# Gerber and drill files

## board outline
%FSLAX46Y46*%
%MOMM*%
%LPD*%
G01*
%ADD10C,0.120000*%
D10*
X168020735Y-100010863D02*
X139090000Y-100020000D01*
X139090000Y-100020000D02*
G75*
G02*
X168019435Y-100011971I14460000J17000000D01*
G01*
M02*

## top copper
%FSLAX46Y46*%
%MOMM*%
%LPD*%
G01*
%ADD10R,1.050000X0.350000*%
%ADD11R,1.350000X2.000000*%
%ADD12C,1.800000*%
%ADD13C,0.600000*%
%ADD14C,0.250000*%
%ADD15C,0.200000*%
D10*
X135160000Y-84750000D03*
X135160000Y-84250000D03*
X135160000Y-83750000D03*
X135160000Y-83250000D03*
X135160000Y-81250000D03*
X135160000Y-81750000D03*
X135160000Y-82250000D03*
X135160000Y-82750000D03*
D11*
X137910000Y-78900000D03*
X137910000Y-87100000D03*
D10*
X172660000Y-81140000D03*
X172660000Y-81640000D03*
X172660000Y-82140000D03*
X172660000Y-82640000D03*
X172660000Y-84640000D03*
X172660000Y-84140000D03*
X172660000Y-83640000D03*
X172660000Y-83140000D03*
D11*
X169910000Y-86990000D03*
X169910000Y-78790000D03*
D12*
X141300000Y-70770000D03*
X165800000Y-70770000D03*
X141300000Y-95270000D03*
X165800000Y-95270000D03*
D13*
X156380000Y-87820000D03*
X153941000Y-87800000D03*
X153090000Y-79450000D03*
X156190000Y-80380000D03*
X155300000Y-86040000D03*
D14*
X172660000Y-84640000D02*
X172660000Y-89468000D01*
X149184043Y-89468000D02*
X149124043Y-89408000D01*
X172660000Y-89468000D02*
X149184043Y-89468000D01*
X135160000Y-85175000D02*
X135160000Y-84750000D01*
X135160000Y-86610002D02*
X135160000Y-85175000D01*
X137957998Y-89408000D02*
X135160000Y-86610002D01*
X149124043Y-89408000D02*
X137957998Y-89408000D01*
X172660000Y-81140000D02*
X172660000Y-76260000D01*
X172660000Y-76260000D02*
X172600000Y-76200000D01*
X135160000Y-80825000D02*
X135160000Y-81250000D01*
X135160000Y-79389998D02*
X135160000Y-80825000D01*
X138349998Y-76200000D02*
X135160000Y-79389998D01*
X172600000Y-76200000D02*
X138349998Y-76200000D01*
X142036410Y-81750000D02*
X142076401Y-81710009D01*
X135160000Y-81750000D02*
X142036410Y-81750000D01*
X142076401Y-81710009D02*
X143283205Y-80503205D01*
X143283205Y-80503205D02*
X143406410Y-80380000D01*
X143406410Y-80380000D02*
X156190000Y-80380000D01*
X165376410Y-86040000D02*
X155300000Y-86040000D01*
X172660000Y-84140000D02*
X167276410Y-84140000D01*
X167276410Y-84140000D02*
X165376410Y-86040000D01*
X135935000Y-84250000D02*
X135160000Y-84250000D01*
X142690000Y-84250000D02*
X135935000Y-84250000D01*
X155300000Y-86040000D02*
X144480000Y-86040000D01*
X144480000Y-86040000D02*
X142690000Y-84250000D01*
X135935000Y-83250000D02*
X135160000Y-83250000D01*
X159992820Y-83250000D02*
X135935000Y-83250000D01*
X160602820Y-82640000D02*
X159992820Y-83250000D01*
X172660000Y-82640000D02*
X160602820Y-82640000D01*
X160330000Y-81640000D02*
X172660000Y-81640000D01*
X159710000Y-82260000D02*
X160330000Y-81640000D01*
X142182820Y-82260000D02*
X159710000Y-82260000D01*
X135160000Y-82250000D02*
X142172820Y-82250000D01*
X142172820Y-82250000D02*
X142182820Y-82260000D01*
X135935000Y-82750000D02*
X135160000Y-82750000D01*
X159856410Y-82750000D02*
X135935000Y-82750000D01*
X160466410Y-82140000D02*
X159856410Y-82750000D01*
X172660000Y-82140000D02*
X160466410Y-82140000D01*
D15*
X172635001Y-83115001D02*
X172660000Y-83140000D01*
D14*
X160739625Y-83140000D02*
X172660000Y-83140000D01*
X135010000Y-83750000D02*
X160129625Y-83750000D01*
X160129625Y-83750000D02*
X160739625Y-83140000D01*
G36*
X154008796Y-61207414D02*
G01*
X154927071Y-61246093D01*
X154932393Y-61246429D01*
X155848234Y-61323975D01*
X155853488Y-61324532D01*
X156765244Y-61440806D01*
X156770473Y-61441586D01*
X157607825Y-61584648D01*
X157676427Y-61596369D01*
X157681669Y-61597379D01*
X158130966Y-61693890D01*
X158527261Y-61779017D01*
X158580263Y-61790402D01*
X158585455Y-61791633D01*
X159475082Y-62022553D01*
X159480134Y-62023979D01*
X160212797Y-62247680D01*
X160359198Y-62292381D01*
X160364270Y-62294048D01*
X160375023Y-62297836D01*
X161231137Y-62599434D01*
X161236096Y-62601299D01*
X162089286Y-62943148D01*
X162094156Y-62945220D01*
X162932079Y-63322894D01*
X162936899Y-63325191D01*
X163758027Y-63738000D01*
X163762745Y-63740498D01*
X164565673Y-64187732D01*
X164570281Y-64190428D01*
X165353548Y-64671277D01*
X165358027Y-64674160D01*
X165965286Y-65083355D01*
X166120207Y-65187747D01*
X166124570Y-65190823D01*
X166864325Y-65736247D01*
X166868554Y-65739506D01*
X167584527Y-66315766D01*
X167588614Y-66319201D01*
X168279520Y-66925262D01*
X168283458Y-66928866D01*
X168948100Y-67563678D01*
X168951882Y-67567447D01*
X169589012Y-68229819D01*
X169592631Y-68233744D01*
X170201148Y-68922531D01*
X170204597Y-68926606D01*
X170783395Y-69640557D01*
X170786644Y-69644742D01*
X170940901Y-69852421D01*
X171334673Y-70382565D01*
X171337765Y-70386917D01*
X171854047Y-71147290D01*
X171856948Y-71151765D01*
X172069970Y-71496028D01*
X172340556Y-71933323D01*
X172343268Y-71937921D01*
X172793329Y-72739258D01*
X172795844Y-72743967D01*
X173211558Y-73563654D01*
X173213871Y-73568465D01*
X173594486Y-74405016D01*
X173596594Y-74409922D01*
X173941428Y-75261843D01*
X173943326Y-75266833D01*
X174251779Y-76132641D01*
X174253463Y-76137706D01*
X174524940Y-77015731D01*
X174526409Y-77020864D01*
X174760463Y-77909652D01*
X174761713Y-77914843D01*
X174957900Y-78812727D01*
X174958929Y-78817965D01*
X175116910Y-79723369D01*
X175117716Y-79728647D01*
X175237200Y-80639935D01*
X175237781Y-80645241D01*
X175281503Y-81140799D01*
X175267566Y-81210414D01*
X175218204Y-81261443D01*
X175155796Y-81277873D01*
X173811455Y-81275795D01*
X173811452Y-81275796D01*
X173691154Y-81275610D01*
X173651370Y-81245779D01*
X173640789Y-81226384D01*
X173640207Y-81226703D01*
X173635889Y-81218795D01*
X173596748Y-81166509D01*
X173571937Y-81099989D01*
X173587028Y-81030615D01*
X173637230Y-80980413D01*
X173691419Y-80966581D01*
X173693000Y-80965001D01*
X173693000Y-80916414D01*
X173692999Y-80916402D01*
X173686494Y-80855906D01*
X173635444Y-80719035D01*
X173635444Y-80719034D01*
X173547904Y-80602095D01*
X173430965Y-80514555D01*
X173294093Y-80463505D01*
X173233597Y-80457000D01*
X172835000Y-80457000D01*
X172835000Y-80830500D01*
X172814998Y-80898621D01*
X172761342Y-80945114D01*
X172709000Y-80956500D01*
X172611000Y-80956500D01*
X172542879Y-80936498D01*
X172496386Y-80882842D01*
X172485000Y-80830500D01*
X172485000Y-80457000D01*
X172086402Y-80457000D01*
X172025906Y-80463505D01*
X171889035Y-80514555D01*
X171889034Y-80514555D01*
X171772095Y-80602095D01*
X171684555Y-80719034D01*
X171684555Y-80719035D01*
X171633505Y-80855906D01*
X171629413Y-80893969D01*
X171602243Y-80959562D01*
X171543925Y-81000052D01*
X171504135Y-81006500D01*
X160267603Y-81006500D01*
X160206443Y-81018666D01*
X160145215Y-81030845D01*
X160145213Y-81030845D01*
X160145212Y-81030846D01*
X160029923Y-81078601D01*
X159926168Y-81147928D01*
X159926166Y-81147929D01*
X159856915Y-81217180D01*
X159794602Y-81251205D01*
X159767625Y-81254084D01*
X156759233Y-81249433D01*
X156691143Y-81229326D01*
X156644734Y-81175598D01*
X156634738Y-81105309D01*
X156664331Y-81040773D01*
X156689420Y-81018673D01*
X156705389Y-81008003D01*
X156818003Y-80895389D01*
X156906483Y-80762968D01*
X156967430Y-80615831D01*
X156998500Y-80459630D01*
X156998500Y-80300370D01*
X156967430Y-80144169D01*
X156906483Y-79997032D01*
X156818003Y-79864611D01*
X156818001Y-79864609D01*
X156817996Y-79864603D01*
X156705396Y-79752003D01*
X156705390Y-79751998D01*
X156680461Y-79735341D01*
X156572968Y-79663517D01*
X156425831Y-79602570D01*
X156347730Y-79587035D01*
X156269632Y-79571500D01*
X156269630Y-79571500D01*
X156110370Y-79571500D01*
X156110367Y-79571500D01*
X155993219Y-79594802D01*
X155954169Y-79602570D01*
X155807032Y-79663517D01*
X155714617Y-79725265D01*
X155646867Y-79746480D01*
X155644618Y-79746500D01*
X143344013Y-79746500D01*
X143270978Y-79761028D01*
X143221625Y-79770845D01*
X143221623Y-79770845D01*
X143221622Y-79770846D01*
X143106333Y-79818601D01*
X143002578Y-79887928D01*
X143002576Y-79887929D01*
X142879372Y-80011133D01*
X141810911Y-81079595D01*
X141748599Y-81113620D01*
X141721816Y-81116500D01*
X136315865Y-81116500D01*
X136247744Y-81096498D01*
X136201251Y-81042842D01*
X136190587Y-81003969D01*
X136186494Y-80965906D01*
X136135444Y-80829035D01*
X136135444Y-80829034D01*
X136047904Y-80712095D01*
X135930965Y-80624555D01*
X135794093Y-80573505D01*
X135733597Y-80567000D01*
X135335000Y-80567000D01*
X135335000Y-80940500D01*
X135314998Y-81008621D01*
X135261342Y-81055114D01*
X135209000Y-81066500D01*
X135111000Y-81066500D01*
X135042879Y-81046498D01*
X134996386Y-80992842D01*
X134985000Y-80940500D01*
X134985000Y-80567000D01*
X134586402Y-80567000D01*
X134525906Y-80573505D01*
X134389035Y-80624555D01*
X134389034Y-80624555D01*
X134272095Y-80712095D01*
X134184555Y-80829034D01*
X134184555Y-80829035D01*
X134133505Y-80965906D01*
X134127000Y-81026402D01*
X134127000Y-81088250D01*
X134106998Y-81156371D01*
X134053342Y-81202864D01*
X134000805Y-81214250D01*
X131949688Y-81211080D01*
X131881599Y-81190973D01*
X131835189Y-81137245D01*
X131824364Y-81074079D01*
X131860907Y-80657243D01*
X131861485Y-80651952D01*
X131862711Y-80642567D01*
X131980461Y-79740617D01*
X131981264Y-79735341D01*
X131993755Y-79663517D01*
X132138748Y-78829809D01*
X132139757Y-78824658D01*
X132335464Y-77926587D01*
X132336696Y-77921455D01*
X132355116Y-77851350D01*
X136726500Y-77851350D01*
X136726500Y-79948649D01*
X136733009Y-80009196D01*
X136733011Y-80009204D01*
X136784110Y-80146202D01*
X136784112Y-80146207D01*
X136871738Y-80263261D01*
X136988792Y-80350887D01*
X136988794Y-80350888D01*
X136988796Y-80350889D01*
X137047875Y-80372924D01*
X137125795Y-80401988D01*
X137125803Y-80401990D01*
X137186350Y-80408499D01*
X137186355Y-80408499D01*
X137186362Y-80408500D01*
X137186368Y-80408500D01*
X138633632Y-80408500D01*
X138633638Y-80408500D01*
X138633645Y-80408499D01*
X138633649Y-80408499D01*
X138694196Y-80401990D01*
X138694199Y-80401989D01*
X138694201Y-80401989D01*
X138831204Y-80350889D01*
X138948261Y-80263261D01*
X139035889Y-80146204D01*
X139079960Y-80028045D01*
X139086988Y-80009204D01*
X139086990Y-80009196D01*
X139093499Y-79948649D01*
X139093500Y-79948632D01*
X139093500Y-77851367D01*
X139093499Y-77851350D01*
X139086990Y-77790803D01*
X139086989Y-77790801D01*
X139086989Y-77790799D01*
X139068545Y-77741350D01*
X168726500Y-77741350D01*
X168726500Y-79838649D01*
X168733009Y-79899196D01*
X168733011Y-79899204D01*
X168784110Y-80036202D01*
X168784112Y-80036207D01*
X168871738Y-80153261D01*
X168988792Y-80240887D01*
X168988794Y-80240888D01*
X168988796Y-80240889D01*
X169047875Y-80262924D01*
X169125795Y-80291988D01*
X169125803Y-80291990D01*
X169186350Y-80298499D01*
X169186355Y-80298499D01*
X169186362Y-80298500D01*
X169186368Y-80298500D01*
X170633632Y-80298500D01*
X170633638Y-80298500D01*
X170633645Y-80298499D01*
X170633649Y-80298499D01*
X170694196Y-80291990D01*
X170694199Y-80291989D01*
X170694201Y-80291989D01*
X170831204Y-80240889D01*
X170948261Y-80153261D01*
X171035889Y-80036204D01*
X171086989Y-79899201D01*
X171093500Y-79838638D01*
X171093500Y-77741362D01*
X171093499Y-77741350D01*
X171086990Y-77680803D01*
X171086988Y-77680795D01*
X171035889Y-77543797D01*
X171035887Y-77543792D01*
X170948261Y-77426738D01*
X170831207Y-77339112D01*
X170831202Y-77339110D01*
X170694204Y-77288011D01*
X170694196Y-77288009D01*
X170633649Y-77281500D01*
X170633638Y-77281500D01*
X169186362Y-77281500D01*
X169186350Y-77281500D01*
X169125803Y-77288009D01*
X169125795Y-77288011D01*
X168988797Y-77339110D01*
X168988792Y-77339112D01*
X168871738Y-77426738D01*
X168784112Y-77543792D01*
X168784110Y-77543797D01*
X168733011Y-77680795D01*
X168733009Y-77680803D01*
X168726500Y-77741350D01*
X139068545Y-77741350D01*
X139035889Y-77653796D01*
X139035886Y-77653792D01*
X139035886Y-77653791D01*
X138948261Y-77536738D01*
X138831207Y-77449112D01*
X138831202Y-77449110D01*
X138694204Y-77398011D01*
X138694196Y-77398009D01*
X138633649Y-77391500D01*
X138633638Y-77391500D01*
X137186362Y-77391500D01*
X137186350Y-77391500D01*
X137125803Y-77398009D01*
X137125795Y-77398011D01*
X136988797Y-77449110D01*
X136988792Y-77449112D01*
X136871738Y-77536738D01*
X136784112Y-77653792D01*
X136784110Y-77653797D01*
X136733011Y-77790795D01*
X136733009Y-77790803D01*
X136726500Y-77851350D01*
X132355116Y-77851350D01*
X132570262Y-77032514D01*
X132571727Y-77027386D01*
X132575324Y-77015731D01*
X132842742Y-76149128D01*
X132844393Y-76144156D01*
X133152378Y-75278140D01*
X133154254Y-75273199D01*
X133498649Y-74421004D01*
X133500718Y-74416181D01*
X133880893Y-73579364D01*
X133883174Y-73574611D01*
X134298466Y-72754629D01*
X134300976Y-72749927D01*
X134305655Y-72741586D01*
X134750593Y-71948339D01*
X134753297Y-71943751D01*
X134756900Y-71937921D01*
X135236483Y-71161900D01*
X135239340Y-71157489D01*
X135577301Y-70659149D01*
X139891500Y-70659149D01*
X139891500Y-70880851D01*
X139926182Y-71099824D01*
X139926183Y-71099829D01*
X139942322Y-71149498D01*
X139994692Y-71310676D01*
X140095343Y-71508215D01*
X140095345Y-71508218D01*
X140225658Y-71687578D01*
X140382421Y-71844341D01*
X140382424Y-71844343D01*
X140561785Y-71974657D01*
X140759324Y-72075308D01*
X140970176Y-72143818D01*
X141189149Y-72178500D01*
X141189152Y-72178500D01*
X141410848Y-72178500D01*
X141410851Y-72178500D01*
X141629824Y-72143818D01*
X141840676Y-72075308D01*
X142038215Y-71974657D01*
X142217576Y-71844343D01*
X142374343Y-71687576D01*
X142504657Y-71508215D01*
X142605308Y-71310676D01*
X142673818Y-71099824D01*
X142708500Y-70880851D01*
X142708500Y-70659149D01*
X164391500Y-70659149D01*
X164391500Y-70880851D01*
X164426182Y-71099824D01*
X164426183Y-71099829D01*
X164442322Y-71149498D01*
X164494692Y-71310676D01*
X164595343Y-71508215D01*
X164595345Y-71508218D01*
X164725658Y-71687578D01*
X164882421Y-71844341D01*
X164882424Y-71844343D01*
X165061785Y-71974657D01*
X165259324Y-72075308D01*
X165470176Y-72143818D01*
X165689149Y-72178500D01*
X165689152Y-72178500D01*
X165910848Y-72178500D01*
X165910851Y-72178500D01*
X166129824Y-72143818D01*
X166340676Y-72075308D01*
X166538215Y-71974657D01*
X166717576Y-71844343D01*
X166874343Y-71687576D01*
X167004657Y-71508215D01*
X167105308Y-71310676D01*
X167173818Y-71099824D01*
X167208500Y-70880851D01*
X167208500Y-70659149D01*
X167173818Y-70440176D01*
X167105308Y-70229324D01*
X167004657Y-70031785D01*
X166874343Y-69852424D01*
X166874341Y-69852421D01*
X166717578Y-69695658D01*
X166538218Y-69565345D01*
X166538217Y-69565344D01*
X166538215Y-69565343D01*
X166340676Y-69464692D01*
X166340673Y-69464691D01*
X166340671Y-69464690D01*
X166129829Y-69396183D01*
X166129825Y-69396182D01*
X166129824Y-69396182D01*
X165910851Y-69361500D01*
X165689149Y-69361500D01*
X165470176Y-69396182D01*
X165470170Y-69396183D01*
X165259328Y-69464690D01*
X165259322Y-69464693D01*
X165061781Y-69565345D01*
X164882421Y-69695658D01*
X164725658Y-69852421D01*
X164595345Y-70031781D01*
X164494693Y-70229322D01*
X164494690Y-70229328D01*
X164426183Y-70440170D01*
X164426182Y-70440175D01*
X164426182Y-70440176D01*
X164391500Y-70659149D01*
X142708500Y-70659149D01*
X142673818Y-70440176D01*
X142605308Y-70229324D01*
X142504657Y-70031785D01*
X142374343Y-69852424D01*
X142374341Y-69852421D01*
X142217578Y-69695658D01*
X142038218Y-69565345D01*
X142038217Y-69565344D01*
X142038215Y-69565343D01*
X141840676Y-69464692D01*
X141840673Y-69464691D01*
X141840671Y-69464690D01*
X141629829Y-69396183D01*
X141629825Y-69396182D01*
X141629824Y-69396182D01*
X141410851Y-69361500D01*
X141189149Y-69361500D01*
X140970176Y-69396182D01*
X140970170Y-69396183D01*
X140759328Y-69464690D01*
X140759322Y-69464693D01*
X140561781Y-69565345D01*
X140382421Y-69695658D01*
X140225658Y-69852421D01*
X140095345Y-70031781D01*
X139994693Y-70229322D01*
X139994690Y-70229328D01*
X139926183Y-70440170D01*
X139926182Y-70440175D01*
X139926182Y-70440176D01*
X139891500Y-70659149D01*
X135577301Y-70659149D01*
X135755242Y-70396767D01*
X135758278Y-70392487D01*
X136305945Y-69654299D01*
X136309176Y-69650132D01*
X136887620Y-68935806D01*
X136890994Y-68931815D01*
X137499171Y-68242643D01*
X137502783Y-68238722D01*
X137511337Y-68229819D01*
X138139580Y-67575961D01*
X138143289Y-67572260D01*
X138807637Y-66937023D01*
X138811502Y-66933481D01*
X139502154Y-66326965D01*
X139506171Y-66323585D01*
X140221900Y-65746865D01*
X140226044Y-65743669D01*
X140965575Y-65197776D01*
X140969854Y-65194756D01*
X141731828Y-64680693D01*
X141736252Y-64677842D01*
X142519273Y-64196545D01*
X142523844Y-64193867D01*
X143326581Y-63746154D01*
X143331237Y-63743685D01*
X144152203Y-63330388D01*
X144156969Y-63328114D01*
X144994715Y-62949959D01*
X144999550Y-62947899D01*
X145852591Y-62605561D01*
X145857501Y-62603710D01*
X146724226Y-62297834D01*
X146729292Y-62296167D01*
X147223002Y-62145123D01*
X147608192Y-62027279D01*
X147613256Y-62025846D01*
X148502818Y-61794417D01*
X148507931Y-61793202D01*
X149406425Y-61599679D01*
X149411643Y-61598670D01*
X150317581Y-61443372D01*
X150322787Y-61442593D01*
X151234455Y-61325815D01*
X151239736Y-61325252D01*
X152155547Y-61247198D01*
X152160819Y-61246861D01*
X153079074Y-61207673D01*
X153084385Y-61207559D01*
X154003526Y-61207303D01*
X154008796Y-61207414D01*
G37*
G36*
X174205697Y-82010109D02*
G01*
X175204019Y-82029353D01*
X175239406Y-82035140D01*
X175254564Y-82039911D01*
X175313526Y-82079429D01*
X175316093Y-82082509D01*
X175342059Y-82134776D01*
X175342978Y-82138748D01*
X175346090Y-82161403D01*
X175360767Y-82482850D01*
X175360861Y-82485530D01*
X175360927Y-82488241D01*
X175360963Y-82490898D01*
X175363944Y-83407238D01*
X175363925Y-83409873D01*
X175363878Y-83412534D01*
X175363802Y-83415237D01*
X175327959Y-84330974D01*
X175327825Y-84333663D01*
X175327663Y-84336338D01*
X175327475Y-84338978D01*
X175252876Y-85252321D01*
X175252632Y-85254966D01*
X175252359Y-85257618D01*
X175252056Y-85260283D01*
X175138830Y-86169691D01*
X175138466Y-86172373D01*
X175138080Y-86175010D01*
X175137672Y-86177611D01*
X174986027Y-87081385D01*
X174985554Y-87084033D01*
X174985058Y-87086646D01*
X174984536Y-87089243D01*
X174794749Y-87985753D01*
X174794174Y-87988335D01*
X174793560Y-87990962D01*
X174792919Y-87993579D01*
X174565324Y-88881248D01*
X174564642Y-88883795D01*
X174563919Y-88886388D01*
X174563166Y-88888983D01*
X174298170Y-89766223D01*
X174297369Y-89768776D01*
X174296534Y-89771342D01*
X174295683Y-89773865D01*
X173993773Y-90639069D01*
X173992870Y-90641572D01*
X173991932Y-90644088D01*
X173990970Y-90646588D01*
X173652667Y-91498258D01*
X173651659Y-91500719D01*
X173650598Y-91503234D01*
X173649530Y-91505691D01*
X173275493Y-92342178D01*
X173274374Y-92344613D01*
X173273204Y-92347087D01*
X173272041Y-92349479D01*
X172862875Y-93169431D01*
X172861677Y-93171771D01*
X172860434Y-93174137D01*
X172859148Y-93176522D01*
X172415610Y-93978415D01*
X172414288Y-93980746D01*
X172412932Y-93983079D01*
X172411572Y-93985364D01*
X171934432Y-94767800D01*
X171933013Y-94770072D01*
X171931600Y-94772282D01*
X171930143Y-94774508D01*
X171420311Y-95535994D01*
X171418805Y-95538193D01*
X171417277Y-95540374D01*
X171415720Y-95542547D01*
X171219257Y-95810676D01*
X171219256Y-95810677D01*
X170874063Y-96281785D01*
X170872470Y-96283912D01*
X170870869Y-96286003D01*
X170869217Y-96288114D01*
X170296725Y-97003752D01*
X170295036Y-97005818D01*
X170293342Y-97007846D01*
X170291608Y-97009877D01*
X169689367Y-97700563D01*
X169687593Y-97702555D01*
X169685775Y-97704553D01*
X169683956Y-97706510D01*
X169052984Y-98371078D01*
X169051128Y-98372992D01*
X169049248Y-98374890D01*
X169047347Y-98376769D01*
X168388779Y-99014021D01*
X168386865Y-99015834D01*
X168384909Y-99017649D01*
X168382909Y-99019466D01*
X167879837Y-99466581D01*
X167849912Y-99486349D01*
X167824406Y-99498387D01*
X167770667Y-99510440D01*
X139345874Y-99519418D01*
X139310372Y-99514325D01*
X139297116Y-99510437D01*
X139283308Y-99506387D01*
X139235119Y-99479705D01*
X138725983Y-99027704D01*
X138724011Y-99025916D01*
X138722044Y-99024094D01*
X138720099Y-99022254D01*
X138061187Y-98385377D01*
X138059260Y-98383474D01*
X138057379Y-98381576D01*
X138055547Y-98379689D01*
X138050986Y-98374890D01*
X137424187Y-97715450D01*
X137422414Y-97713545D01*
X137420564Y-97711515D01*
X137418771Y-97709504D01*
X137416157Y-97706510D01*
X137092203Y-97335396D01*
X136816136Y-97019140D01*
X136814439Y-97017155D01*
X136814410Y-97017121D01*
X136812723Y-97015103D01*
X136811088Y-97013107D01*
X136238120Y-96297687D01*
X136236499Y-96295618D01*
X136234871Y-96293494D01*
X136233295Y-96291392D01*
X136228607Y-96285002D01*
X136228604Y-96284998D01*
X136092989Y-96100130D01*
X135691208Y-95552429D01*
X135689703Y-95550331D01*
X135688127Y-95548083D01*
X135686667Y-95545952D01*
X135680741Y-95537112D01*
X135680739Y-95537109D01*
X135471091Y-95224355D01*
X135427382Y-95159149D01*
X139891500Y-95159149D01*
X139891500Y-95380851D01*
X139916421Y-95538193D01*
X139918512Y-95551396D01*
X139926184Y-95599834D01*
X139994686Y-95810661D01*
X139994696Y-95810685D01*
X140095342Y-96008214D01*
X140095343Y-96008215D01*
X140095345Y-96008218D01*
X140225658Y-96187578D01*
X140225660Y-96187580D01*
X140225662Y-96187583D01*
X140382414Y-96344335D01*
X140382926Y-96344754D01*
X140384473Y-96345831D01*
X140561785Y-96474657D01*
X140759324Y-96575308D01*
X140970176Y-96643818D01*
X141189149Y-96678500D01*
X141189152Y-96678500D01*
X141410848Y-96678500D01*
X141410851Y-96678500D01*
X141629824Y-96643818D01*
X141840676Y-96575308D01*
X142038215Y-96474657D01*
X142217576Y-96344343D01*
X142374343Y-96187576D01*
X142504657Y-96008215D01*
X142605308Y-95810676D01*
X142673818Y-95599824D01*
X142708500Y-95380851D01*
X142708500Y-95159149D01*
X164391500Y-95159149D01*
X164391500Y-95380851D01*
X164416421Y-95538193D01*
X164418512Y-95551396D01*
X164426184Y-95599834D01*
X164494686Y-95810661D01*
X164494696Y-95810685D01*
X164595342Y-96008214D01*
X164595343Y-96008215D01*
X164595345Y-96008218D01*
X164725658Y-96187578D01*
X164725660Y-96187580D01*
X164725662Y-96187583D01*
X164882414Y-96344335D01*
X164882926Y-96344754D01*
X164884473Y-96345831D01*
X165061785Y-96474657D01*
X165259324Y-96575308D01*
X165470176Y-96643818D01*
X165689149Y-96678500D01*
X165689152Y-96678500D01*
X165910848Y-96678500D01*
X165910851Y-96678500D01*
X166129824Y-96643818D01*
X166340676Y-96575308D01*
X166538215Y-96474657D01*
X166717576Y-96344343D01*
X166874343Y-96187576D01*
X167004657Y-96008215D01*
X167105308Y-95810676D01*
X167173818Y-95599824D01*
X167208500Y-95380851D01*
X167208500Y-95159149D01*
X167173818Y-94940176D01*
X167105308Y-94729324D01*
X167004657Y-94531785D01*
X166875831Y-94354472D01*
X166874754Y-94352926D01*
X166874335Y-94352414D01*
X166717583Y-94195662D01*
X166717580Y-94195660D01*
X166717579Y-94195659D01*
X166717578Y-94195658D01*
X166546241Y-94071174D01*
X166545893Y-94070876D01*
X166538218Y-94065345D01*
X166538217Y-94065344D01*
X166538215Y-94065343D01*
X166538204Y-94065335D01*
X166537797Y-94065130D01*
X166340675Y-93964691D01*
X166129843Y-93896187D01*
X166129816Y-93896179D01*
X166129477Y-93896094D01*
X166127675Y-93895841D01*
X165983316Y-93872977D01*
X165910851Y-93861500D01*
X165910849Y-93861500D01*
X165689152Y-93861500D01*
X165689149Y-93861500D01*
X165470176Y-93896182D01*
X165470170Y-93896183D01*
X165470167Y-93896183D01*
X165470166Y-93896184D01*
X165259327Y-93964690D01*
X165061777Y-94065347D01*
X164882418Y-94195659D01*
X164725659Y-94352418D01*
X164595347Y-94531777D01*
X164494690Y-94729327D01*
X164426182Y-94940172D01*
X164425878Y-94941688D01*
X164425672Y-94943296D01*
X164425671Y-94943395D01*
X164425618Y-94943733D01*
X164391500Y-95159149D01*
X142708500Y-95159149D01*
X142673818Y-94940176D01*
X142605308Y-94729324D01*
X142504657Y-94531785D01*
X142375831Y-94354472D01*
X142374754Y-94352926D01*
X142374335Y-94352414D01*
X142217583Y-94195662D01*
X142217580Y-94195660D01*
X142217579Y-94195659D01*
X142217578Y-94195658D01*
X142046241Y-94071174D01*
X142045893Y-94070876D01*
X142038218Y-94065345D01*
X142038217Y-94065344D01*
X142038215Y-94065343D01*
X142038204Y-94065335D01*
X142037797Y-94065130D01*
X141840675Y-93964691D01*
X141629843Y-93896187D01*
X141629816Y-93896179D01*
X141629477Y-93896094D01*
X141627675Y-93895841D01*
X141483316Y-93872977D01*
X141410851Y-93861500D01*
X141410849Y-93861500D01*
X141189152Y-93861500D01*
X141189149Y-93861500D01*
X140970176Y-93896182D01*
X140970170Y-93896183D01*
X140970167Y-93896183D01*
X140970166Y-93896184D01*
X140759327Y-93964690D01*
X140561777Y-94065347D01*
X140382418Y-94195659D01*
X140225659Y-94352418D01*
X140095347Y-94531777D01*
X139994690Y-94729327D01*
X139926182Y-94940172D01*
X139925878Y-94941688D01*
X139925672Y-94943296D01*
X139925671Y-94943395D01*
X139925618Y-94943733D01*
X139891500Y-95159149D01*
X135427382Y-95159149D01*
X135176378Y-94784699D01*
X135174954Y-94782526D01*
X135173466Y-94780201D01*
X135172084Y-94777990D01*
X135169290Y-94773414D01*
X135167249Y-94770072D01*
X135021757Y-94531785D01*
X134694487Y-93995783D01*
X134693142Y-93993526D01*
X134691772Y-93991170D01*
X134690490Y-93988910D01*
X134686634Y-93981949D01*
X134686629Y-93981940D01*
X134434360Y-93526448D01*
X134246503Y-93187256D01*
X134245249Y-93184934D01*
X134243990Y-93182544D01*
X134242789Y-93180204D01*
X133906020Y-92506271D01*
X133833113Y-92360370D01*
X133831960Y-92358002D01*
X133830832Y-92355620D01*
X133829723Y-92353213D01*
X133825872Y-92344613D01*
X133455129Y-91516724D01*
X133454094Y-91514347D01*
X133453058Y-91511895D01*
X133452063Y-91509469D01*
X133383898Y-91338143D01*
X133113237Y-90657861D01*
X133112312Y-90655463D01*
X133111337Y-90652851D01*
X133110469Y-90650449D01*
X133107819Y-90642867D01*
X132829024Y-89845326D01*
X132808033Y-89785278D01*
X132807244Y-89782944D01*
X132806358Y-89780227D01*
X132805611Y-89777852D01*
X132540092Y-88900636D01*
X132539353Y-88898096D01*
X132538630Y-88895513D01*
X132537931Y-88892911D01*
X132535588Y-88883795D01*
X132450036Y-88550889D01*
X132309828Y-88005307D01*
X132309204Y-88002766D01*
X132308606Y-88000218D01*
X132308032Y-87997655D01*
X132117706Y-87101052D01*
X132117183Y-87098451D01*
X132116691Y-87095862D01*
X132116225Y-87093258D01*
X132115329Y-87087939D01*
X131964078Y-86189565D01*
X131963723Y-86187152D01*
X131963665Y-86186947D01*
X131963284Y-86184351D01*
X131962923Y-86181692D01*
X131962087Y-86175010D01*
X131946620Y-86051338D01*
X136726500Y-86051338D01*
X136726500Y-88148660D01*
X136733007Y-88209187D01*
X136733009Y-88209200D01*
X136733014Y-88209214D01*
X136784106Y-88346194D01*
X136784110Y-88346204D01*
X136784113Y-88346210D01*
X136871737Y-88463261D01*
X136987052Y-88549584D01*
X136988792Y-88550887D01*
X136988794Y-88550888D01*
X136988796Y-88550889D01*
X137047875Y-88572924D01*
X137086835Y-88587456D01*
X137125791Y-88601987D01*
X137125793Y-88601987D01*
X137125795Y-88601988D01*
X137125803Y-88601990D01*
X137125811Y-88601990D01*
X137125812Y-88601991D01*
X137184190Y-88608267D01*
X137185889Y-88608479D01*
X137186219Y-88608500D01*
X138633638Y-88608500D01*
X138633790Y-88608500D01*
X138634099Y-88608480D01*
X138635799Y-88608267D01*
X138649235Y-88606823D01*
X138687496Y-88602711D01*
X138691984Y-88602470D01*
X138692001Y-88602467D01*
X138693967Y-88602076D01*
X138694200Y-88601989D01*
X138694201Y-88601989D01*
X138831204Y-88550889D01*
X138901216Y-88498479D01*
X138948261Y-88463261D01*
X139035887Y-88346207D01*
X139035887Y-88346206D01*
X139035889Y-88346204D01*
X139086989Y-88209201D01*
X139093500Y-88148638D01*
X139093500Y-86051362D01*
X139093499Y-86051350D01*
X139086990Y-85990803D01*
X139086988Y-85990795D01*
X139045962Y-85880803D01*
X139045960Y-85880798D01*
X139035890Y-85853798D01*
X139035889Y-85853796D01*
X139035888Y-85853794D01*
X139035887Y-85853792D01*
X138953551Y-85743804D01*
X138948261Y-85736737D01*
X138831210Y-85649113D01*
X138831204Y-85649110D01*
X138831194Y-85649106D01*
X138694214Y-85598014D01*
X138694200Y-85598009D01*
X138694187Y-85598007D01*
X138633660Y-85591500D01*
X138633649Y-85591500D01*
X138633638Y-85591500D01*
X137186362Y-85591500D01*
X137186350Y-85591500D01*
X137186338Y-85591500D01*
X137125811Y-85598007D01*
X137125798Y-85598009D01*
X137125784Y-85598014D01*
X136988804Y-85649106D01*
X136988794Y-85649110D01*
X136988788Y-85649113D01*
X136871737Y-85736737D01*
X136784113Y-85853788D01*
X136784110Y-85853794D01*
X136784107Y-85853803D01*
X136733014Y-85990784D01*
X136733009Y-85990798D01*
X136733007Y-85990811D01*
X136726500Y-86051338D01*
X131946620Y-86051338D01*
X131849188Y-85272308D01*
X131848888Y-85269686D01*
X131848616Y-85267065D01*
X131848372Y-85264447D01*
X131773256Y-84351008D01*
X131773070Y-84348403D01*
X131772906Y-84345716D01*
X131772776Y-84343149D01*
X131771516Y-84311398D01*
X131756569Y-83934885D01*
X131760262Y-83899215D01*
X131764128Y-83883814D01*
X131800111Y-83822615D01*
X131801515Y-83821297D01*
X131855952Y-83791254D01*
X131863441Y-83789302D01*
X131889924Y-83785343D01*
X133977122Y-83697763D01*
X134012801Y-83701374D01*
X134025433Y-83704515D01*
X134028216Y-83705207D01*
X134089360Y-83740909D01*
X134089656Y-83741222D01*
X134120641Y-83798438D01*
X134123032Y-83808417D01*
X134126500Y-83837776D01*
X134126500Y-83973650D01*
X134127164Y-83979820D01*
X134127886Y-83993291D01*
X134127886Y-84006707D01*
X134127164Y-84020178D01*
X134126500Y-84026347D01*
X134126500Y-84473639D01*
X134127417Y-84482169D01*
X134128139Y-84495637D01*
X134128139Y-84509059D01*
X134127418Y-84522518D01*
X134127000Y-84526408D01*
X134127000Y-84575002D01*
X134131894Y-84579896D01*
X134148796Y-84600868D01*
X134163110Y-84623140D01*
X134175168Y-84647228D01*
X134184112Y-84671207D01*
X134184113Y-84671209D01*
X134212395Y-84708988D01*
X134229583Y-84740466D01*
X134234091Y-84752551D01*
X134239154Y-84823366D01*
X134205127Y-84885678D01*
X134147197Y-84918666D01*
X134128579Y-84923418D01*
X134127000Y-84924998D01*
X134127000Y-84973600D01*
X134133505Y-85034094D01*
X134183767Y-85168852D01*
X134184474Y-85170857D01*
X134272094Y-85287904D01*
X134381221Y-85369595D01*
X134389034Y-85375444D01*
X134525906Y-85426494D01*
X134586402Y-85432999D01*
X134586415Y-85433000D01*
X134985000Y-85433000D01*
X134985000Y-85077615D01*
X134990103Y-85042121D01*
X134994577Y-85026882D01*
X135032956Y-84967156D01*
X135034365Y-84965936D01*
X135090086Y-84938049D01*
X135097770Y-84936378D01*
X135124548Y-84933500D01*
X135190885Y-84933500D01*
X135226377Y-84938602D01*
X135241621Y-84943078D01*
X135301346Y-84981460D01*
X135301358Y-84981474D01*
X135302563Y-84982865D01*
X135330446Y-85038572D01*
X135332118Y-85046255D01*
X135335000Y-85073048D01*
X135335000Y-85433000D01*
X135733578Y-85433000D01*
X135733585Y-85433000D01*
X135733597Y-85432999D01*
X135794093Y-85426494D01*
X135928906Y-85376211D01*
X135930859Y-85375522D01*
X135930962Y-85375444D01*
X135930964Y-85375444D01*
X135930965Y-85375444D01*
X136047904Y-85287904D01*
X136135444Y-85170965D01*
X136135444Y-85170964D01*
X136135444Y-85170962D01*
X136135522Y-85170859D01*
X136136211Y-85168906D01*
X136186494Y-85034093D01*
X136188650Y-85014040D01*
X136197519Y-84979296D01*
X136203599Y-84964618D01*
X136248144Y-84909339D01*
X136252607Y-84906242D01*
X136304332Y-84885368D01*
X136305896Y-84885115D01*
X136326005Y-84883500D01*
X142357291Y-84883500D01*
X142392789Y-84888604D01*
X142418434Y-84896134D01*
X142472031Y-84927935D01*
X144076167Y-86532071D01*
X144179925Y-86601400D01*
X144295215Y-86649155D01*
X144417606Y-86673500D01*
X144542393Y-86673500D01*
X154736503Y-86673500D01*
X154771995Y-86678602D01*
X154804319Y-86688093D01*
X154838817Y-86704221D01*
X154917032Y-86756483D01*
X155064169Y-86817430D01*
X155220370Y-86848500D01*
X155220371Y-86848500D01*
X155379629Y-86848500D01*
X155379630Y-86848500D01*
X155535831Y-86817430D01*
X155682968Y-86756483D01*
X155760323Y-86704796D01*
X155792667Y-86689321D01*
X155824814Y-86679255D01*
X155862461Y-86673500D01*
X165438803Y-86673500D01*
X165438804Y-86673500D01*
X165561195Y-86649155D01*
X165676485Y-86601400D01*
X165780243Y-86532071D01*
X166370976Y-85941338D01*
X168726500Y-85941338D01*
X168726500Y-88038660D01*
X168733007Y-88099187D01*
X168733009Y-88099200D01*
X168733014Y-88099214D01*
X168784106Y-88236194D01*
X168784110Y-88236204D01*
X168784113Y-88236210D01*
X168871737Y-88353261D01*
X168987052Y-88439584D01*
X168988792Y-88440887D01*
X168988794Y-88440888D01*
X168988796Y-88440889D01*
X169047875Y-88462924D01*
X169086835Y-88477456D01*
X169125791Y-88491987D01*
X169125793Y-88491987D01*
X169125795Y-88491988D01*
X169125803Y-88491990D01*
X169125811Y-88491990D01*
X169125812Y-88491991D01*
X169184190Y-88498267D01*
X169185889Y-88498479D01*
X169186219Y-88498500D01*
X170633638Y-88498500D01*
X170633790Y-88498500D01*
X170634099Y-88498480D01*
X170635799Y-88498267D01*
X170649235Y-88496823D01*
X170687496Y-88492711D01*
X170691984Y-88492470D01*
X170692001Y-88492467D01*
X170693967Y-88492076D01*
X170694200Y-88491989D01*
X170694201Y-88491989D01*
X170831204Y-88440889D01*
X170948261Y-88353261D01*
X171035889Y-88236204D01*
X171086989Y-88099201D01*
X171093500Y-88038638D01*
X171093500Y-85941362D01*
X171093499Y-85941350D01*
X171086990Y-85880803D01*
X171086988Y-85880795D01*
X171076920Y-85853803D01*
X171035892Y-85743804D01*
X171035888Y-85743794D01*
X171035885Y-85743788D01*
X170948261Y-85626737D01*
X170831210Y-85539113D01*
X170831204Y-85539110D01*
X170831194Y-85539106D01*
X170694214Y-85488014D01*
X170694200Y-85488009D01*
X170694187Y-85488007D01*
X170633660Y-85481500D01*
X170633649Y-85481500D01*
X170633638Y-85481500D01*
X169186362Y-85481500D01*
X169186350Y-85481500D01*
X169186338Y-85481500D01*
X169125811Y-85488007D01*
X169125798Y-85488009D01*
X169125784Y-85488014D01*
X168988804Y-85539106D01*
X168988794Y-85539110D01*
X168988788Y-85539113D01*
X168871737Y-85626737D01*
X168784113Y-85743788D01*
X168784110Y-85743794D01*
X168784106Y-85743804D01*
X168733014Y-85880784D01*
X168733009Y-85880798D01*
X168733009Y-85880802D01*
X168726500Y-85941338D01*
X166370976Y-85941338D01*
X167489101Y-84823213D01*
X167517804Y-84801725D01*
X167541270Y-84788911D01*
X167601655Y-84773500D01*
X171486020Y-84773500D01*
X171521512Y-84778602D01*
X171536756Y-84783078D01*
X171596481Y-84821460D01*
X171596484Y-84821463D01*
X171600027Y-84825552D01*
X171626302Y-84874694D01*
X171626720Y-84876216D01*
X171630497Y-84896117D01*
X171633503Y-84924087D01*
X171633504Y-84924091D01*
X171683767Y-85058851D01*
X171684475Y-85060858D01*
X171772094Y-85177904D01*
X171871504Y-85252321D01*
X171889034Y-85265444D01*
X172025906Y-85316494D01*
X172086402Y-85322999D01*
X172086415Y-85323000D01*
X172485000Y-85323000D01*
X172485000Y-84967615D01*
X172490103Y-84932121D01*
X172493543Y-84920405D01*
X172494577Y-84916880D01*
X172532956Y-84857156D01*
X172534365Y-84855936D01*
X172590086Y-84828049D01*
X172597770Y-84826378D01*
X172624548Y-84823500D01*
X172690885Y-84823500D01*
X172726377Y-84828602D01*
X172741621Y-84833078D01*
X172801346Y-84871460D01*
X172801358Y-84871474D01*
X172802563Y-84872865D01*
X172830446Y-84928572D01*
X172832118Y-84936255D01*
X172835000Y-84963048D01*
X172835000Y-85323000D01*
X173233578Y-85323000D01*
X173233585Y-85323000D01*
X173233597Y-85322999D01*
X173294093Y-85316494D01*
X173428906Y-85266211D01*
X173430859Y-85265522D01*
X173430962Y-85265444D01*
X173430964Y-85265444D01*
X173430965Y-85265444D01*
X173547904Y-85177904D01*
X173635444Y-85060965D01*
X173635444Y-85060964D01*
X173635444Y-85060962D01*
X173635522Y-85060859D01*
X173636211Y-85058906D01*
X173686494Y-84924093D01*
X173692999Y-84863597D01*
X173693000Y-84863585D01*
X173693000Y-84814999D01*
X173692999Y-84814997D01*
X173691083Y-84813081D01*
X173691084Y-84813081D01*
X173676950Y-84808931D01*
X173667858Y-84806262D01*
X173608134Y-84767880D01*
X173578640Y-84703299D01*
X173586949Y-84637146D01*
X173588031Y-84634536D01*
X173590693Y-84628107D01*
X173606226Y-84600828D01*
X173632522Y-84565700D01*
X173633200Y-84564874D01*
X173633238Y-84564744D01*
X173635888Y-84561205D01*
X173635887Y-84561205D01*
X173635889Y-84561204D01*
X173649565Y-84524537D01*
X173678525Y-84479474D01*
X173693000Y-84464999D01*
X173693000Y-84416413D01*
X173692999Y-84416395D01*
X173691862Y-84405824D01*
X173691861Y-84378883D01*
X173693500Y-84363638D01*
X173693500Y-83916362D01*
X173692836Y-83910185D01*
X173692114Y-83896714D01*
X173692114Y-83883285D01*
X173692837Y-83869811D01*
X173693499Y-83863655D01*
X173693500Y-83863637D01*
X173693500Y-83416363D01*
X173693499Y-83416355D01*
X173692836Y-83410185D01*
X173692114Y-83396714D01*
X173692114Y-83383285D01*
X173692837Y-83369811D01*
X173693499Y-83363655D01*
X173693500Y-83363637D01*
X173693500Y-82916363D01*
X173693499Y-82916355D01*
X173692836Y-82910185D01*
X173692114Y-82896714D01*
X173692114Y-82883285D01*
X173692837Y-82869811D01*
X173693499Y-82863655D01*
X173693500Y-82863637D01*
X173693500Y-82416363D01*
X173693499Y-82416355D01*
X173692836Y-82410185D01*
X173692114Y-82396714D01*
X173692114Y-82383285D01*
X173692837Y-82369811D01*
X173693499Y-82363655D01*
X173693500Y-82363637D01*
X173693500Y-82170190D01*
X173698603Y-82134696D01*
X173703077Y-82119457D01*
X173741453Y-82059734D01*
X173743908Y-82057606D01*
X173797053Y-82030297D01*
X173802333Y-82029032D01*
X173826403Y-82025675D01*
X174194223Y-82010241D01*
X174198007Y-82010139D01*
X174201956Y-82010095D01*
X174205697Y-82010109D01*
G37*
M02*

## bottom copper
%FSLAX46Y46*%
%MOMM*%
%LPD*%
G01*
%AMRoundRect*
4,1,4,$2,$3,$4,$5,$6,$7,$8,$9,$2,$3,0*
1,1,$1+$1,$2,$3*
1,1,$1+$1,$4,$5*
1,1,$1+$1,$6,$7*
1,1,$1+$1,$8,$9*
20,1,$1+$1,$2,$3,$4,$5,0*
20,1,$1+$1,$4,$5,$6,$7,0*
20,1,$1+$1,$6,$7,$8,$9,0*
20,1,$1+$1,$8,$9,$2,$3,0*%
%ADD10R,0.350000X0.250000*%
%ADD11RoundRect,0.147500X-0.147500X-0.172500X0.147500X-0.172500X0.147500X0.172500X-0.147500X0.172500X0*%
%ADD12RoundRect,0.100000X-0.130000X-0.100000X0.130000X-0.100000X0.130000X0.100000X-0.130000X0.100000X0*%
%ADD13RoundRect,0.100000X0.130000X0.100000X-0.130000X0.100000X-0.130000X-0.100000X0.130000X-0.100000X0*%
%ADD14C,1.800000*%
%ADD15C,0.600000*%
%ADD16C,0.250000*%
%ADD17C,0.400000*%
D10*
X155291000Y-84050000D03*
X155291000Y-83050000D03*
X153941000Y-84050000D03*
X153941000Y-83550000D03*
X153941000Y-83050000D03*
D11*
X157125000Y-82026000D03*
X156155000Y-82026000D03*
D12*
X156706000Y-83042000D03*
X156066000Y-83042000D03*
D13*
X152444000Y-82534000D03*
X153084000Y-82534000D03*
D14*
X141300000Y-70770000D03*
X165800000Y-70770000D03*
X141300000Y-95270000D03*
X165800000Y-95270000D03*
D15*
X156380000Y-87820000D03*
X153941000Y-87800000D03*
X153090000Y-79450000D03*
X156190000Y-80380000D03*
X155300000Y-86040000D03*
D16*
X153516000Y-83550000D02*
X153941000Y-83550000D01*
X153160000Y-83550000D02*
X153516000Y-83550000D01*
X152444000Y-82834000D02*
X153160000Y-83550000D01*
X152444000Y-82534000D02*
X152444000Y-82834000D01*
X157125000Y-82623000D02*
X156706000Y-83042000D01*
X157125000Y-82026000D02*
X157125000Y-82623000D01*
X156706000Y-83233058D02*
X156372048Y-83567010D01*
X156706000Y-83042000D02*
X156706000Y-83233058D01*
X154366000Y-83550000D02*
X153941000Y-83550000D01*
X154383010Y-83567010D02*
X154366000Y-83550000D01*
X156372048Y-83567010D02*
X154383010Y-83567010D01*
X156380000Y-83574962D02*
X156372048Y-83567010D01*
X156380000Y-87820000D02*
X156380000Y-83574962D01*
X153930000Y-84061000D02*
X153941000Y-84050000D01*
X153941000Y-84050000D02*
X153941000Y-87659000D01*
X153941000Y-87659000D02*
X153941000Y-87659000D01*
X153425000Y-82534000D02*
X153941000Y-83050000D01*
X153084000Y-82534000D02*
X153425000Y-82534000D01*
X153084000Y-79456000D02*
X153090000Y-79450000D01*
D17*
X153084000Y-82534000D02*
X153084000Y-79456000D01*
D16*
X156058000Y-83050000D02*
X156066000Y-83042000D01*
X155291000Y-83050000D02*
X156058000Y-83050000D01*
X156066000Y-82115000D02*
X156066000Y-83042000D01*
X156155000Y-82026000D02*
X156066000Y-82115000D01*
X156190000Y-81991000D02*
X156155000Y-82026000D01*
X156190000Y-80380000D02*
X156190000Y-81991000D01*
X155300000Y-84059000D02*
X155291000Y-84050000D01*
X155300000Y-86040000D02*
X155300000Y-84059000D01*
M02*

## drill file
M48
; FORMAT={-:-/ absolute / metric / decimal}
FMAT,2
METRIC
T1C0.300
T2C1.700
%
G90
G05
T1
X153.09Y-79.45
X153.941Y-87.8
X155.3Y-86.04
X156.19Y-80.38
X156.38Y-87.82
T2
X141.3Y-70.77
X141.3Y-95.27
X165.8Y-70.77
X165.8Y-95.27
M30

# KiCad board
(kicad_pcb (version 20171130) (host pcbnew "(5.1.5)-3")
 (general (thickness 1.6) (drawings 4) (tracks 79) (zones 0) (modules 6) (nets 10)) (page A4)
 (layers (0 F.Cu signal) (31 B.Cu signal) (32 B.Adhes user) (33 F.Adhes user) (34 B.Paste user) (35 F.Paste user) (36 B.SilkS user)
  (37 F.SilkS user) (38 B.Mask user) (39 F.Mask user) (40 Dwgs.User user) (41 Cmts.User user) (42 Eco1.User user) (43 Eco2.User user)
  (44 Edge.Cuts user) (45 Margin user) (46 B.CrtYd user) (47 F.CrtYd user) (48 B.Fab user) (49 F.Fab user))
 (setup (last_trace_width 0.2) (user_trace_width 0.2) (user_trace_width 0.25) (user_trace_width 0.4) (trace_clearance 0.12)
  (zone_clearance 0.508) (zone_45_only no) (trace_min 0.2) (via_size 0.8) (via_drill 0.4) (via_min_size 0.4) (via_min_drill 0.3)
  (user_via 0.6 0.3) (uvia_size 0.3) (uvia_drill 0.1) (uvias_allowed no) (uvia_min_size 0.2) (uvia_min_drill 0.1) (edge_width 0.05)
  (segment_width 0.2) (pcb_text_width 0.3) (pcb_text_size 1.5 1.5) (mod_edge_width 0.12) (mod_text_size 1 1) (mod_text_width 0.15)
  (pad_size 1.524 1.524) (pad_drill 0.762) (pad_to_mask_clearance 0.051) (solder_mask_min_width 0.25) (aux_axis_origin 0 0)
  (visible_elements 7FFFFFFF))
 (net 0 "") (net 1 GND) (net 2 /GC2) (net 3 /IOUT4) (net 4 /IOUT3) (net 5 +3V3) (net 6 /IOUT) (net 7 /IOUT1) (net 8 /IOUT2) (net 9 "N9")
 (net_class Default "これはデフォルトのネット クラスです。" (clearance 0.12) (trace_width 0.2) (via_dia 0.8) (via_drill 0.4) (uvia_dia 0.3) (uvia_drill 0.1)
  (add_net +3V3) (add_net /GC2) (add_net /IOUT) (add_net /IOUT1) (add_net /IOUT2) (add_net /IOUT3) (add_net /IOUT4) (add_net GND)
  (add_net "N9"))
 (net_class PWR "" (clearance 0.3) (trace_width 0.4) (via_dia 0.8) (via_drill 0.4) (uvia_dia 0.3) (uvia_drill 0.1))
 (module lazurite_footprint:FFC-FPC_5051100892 (layer F.Cu) (at 135.685 83 90)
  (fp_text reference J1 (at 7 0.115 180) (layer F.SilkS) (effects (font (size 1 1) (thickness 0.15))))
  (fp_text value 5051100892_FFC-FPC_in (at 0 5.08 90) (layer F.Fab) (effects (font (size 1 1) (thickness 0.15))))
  (pad 1 smd rect (at -1.75 -0.525 90) (size 0.35 1.05) (layers F.Cu F.Paste F.Mask) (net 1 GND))
  (pad 2 smd rect (at -1.25 -0.525 90) (size 0.35 1.05) (layers F.Cu F.Paste F.Mask) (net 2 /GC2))
  (pad 3 smd rect (at -0.75 -0.525 90) (size 0.35 1.05) (layers F.Cu F.Paste F.Mask) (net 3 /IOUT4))
  (pad 4 smd rect (at -0.25 -0.525 90) (size 0.35 1.05) (layers F.Cu F.Paste F.Mask) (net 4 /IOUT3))
  (pad 8 smd rect (at 1.75 -0.525 90) (size 0.35 1.05) (layers F.Cu F.Paste F.Mask) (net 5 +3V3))
  (pad 7 smd rect (at 1.25 -0.525 90) (size 0.35 1.05) (layers F.Cu F.Paste F.Mask) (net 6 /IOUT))
  (pad 6 smd rect (at 0.75 -0.525 90) (size 0.35 1.05) (layers F.Cu F.Paste F.Mask) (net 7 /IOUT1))
  (pad 5 smd rect (at 0.25 -0.525 90) (size 0.35 1.05) (layers F.Cu F.Paste F.Mask) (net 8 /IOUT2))
  (pad 9 smd rect (at 4.1 2.225 90) (size 2 1.35) (layers F.Cu F.Paste F.Mask))
  (pad 9 smd rect (at -4.1 2.225 90) (size 2 1.35) (layers F.Cu F.Paste F.Mask)))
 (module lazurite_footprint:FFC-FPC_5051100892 (layer F.Cu) (at 172.135 82.89 270)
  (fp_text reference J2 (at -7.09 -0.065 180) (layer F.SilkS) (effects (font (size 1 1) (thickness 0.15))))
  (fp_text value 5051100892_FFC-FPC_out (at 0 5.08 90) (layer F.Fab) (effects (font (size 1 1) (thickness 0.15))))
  (pad 1 smd rect (at -1.75 -0.525 270) (size 0.35 1.05) (layers F.Cu F.Paste F.Mask) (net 5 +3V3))
  (pad 2 smd rect (at -1.25 -0.525 270) (size 0.35 1.05) (layers F.Cu F.Paste F.Mask) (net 7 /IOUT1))
  (pad 3 smd rect (at -0.75 -0.525 270) (size 0.35 1.05) (layers F.Cu F.Paste F.Mask) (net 8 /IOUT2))
  (pad 4 smd rect (at -0.25 -0.525 270) (size 0.35 1.05) (layers F.Cu F.Paste F.Mask) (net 4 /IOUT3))
  (pad 8 smd rect (at 1.75 -0.525 270) (size 0.35 1.05) (layers F.Cu F.Paste F.Mask) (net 1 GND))
  (pad 7 smd rect (at 1.25 -0.525 270) (size 0.35 1.05) (layers F.Cu F.Paste F.Mask) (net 2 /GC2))
  (pad 6 smd rect (at 0.75 -0.525 270) (size 0.35 1.05) (layers F.Cu F.Paste F.Mask) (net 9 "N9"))
  (pad 5 smd rect (at 0.25 -0.525 270) (size 0.35 1.05) (layers F.Cu F.Paste F.Mask) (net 3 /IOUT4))
  (pad 9 smd rect (at 4.1 2.225 270) (size 2 1.35) (layers F.Cu F.Paste F.Mask))
  (pad 9 smd rect (at -4.1 2.225 270) (size 2 1.35) (layers F.Cu F.Paste F.Mask)))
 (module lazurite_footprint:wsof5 (layer B.Cu) (at 155.116 83.55 270)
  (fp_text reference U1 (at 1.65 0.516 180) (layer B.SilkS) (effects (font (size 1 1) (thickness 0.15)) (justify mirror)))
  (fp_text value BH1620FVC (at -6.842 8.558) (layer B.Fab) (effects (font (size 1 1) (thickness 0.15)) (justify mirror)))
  (pad 4 smd rect (at 0.5 -0.175 270) (size 0.25 0.35) (layers B.Cu B.Paste B.Mask) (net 2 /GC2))
  (pad 5 smd rect (at -0.5 -0.175 270) (size 0.25 0.35) (layers B.Cu B.Paste B.Mask) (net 6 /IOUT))
  (pad 3 smd rect (at 0.5 1.175 270) (size 0.25 0.35) (layers B.Cu B.Paste B.Mask) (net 1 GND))
  (pad 2 smd rect (at 0 1.175 270) (size 0.25 0.35) (layers B.Cu B.Paste B.Mask) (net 1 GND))
  (pad 1 smd rect (at -0.5 1.175 270) (size 0.25 0.35) (layers B.Cu B.Paste B.Mask) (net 5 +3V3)))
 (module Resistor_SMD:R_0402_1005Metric (layer B.Cu) (at 156.64 82.026)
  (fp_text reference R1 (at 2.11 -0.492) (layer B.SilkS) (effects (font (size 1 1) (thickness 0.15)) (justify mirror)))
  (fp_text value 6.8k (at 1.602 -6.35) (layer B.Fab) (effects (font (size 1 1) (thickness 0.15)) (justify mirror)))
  (pad 2 smd roundrect (at 0.485 0) (size 0.59 0.64) (layers B.Cu B.Paste B.Mask) (roundrect_rratio 0.25) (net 1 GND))
  (pad 1 smd roundrect (at -0.485 0) (size 0.59 0.64) (layers B.Cu B.Paste B.Mask) (roundrect_rratio 0.25) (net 6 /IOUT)))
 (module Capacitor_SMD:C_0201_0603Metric (layer B.Cu) (at 156.386 83.042)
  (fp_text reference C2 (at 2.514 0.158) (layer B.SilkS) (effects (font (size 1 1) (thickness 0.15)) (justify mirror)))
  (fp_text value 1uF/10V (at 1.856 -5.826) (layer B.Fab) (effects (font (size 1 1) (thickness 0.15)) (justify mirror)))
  (pad 2 smd roundrect (at 0.32 0) (size 0.46 0.4) (layers B.Cu B.Mask) (roundrect_rratio 0.25) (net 1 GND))
  (pad 1 smd roundrect (at -0.32 0) (size 0.46 0.4) (layers B.Cu B.Mask) (roundrect_rratio 0.25) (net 6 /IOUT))
  (pad "" smd roundrect (at 0.345 0) (size 0.318 0.36) (layers B.Paste) (roundrect_rratio 0.25))
  (pad "" smd roundrect (at -0.345 0) (size 0.318 0.36) (layers B.Paste) (roundrect_rratio 0.25)))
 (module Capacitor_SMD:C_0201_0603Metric (layer B.Cu) (at 152.764 82.534 180)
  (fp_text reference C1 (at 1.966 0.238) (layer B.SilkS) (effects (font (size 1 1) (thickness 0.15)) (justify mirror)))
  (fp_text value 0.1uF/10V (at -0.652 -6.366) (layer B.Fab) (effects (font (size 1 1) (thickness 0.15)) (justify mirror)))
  (pad 2 smd roundrect (at 0.32 0 180) (size 0.46 0.4) (layers B.Cu B.Mask) (roundrect_rratio 0.25) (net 1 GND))
  (pad 1 smd roundrect (at -0.32 0 180) (size 0.46 0.4) (layers B.Cu B.Mask) (roundrect_rratio 0.25) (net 5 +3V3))
  (pad "" smd roundrect (at 0.345 0 180) (size 0.318 0.36) (layers B.Paste) (roundrect_rratio 0.25))
  (pad "" smd roundrect (at -0.345 0 180) (size 0.318 0.36) (layers B.Paste) (roundrect_rratio 0.25)))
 (gr_line (start 168.020735 100.010863) (end 139.09 100.02) (layer Edge.Cuts) (width 0.12))
 (gr_arc (start 153.55 83.02) (end 139.09 100.02) (angle 279.2) (layer Edge.Cuts) (width 0.12))
 (via (at 141.3 70.77) (size 1.8) (drill 1.7) (layers F.Cu B.Cu) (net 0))
 (via (at 165.8 70.77) (size 1.8) (drill 1.7) (layers F.Cu B.Cu) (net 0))
 (via (at 141.3 95.27) (size 1.8) (drill 1.7) (layers F.Cu B.Cu) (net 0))
 (via (at 165.8 95.27) (size 1.8) (drill 1.7) (layers F.Cu B.Cu) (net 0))
 (segment (start 153.516 83.55) (end 153.941 83.55) (width 0.25) (layer B.Cu) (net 1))
 (segment (start 153.16 83.55) (end 153.516 83.55) (width 0.25) (layer B.Cu) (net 1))
 (segment (start 152.444 82.834) (end 153.16 83.55) (width 0.25) (layer B.Cu) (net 1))
 (segment (start 152.444 82.534) (end 152.444 82.834) (width 0.25) (layer B.Cu) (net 1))
 (segment (start 157.125 82.623) (end 156.706 83.042) (width 0.25) (layer B.Cu) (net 1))
 (segment (start 157.125 82.026) (end 157.125 82.623) (width 0.25) (layer B.Cu) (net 1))
 (segment (start 156.706 83.233058) (end 156.372048 83.56701) (width 0.25) (layer B.Cu) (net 1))
 (segment (start 156.706 83.042) (end 156.706 83.233058) (width 0.25) (layer B.Cu) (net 1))
 (segment (start 154.366 83.55) (end 153.941 83.55) (width 0.25) (layer B.Cu) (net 1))
 (segment (start 154.38301 83.56701) (end 154.366 83.55) (width 0.25) (layer B.Cu) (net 1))
 (segment (start 156.372048 83.56701) (end 154.38301 83.56701) (width 0.25) (layer B.Cu) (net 1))
 (via (at 156.38 87.82) (size 0.6) (drill 0.3) (layers F.Cu B.Cu) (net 1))
 (segment (start 156.38 83.574962) (end 156.372048 83.56701) (width 0.25) (layer B.Cu) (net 1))
 (segment (start 156.38 87.82) (end 156.38 83.574962) (width 0.25) (layer B.Cu) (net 1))
 (segment (start 172.66 84.64) (end 172.66 89.468) (width 0.25) (layer F.Cu) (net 1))
 (segment (start 149.184043 89.468) (end 149.124043 89.408) (width 0.25) (layer F.Cu) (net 1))
 (segment (start 172.66 89.468) (end 149.184043 89.468) (width 0.25) (layer F.Cu) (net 1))
 (segment (start 135.16 85.175) (end 135.16 84.75) (width 0.25) (layer F.Cu) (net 1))
 (segment (start 135.16 86.610002) (end 135.16 85.175) (width 0.25) (layer F.Cu) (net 1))
 (segment (start 137.957998 89.408) (end 135.16 86.610002) (width 0.25) (layer F.Cu) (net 1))
 (segment (start 149.124043 89.408) (end 137.957998 89.408) (width 0.25) (layer F.Cu) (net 1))
 (segment (start 153.93 84.061) (end 153.941 84.05) (width 0.25) (layer B.Cu) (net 1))
 (segment (start 153.941 84.05) (end 153.941 87.659) (width 0.25) (layer B.Cu) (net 1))
 (segment (start 153.941 87.659) (end 153.941 87.659) (width 0.25) (layer B.Cu) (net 1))
 (via (at 153.941 87.8) (size 0.6) (drill 0.3) (layers F.Cu B.Cu) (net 1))
 (segment (start 153.425 82.534) (end 153.941 83.05) (width 0.25) (layer B.Cu) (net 5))
 (segment (start 153.084 82.534) (end 153.425 82.534) (width 0.25) (layer B.Cu) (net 5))
 (via (at 153.09 79.45) (size 0.6) (drill 0.3) (layers F.Cu B.Cu) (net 5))
 (segment (start 153.084 79.456) (end 153.09 79.45) (width 0.25) (layer B.Cu) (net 5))
 (segment (start 153.084 82.534) (end 153.084 79.456) (width 0.4) (layer B.Cu) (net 5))
 (segment (start 172.66 81.14) (end 172.66 76.26) (width 0.25) (layer F.Cu) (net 5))
 (segment (start 172.66 76.26) (end 172.6 76.2) (width 0.25) (layer F.Cu) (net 5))
 (segment (start 135.16 80.825) (end 135.16 81.25) (width 0.25) (layer F.Cu) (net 5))
 (segment (start 135.16 79.389998) (end 135.16 80.825) (width 0.25) (layer F.Cu) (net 5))
 (segment (start 138.349998 76.2) (end 135.16 79.389998) (width 0.25) (layer F.Cu) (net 5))
 (segment (start 172.6 76.2) (end 138.349998 76.2) (width 0.25) (layer F.Cu) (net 5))
 (segment (start 156.058 83.05) (end 156.066 83.042) (width 0.25) (layer B.Cu) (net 6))
 (segment (start 155.291 83.05) (end 156.058 83.05) (width 0.25) (layer B.Cu) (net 6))
 (segment (start 156.066 82.115) (end 156.066 83.042) (width 0.25) (layer B.Cu) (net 6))
 (segment (start 156.155 82.026) (end 156.066 82.115) (width 0.25) (layer B.Cu) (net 6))
 (segment (start 142.03641 81.75) (end 142.076401 81.710009) (width 0.25) (layer F.Cu) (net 6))
 (segment (start 135.16 81.75) (end 142.03641 81.75) (width 0.25) (layer F.Cu) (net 6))
 (segment (start 142.076401 81.710009) (end 143.283205 80.503205) (width 0.25) (layer F.Cu) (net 6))
 (via (at 156.19 80.38) (size 0.6) (drill 0.3) (layers F.Cu B.Cu) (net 6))
 (segment (start 143.283205 80.503205) (end 143.40641 80.38) (width 0.25) (layer F.Cu) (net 6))
 (segment (start 143.40641 80.38) (end 156.19 80.38) (width 0.25) (layer F.Cu) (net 6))
 (segment (start 156.19 81.991) (end 156.155 82.026) (width 0.25) (layer B.Cu) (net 6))
 (segment (start 156.19 80.38) (end 156.19 81.991) (width 0.25) (layer B.Cu) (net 6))
 (via (at 155.3 86.04) (size 0.6) (drill 0.3) (layers F.Cu B.Cu) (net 2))
 (segment (start 165.37641 86.04) (end 155.3 86.04) (width 0.25) (layer F.Cu) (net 2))
 (segment (start 172.66 84.14) (end 167.27641 84.14) (width 0.25) (layer F.Cu) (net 2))
 (segment (start 167.27641 84.14) (end 165.37641 86.04) (width 0.25) (layer F.Cu) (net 2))
 (segment (start 155.3 84.059) (end 155.291 84.05) (width 0.25) (layer B.Cu) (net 2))
 (segment (start 155.3 86.04) (end 155.3 84.059) (width 0.25) (layer B.Cu) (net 2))
 (segment (start 135.935 84.25) (end 135.16 84.25) (width 0.25) (layer F.Cu) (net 2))
 (segment (start 142.69 84.25) (end 135.935 84.25) (width 0.25) (layer F.Cu) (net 2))
 (segment (start 155.3 86.04) (end 144.48 86.04) (width 0.25) (layer F.Cu) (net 2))
 (segment (start 144.48 86.04) (end 142.69 84.25) (width 0.25) (layer F.Cu) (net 2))
 (segment (start 135.935 83.25) (end 135.16 83.25) (width 0.25) (layer F.Cu) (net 4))
 (segment (start 159.99282 83.25) (end 135.935 83.25) (width 0.25) (layer F.Cu) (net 4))
 (segment (start 160.60282 82.64) (end 159.99282 83.25) (width 0.25) (layer F.Cu) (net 4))
 (segment (start 172.66 82.64) (end 160.60282 82.64) (width 0.25) (layer F.Cu) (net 4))
 (segment (start 160.33 81.64) (end 172.66 81.64) (width 0.25) (layer F.Cu) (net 7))
 (segment (start 159.71 82.26) (end 160.33 81.64) (width 0.25) (layer F.Cu) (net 7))
 (segment (start 142.18282 82.26) (end 159.71 82.26) (width 0.25) (layer F.Cu) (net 7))
 (segment (start 135.16 82.25) (end 142.17282 82.25) (width 0.25) (layer F.Cu) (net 7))
 (segment (start 142.17282 82.25) (end 142.18282 82.26) (width 0.25) (layer F.Cu) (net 7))
 (segment (start 135.935 82.75) (end 135.16 82.75) (width 0.25) (layer F.Cu) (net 8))
 (segment (start 159.85641 82.75) (end 135.935 82.75) (width 0.25) (layer F.Cu) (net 8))
 (segment (start 160.46641 82.14) (end 159.85641 82.75) (width 0.25) (layer F.Cu) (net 8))
 (segment (start 172.66 82.14) (end 160.46641 82.14) (width 0.25) (layer F.Cu) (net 8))
 (segment (start 172.635001 83.115001) (end 172.66 83.14) (width 0.2) (layer F.Cu) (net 3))
 (segment (start 160.739625 83.14) (end 172.66 83.14) (width 0.25) (layer F.Cu) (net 3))
 (segment (start 135.01 83.75) (end 160.129625 83.75) (width 0.25) (layer F.Cu) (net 3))
 (segment (start 160.129625 83.75) (end 160.739625 83.14) (width 0.25) (layer F.Cu) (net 3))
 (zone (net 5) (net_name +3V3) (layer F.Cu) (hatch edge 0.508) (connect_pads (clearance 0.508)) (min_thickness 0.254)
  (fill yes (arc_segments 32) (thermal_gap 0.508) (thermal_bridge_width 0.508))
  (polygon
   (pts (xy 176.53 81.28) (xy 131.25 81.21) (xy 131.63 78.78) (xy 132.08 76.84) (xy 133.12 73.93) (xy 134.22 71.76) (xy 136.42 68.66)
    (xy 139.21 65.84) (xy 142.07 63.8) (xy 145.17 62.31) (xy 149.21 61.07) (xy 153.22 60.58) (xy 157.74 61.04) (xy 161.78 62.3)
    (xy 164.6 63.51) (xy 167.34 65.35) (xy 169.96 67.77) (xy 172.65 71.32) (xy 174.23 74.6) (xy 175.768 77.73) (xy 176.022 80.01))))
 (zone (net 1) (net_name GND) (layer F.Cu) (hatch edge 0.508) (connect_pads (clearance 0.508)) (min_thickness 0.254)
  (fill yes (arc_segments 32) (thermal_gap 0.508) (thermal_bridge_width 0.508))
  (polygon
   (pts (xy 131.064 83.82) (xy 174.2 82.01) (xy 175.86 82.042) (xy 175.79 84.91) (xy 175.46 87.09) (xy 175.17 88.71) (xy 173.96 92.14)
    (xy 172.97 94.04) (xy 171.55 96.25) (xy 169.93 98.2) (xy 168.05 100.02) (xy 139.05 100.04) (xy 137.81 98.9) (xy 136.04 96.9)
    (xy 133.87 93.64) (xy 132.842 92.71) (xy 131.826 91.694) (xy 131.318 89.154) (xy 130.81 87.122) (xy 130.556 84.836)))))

